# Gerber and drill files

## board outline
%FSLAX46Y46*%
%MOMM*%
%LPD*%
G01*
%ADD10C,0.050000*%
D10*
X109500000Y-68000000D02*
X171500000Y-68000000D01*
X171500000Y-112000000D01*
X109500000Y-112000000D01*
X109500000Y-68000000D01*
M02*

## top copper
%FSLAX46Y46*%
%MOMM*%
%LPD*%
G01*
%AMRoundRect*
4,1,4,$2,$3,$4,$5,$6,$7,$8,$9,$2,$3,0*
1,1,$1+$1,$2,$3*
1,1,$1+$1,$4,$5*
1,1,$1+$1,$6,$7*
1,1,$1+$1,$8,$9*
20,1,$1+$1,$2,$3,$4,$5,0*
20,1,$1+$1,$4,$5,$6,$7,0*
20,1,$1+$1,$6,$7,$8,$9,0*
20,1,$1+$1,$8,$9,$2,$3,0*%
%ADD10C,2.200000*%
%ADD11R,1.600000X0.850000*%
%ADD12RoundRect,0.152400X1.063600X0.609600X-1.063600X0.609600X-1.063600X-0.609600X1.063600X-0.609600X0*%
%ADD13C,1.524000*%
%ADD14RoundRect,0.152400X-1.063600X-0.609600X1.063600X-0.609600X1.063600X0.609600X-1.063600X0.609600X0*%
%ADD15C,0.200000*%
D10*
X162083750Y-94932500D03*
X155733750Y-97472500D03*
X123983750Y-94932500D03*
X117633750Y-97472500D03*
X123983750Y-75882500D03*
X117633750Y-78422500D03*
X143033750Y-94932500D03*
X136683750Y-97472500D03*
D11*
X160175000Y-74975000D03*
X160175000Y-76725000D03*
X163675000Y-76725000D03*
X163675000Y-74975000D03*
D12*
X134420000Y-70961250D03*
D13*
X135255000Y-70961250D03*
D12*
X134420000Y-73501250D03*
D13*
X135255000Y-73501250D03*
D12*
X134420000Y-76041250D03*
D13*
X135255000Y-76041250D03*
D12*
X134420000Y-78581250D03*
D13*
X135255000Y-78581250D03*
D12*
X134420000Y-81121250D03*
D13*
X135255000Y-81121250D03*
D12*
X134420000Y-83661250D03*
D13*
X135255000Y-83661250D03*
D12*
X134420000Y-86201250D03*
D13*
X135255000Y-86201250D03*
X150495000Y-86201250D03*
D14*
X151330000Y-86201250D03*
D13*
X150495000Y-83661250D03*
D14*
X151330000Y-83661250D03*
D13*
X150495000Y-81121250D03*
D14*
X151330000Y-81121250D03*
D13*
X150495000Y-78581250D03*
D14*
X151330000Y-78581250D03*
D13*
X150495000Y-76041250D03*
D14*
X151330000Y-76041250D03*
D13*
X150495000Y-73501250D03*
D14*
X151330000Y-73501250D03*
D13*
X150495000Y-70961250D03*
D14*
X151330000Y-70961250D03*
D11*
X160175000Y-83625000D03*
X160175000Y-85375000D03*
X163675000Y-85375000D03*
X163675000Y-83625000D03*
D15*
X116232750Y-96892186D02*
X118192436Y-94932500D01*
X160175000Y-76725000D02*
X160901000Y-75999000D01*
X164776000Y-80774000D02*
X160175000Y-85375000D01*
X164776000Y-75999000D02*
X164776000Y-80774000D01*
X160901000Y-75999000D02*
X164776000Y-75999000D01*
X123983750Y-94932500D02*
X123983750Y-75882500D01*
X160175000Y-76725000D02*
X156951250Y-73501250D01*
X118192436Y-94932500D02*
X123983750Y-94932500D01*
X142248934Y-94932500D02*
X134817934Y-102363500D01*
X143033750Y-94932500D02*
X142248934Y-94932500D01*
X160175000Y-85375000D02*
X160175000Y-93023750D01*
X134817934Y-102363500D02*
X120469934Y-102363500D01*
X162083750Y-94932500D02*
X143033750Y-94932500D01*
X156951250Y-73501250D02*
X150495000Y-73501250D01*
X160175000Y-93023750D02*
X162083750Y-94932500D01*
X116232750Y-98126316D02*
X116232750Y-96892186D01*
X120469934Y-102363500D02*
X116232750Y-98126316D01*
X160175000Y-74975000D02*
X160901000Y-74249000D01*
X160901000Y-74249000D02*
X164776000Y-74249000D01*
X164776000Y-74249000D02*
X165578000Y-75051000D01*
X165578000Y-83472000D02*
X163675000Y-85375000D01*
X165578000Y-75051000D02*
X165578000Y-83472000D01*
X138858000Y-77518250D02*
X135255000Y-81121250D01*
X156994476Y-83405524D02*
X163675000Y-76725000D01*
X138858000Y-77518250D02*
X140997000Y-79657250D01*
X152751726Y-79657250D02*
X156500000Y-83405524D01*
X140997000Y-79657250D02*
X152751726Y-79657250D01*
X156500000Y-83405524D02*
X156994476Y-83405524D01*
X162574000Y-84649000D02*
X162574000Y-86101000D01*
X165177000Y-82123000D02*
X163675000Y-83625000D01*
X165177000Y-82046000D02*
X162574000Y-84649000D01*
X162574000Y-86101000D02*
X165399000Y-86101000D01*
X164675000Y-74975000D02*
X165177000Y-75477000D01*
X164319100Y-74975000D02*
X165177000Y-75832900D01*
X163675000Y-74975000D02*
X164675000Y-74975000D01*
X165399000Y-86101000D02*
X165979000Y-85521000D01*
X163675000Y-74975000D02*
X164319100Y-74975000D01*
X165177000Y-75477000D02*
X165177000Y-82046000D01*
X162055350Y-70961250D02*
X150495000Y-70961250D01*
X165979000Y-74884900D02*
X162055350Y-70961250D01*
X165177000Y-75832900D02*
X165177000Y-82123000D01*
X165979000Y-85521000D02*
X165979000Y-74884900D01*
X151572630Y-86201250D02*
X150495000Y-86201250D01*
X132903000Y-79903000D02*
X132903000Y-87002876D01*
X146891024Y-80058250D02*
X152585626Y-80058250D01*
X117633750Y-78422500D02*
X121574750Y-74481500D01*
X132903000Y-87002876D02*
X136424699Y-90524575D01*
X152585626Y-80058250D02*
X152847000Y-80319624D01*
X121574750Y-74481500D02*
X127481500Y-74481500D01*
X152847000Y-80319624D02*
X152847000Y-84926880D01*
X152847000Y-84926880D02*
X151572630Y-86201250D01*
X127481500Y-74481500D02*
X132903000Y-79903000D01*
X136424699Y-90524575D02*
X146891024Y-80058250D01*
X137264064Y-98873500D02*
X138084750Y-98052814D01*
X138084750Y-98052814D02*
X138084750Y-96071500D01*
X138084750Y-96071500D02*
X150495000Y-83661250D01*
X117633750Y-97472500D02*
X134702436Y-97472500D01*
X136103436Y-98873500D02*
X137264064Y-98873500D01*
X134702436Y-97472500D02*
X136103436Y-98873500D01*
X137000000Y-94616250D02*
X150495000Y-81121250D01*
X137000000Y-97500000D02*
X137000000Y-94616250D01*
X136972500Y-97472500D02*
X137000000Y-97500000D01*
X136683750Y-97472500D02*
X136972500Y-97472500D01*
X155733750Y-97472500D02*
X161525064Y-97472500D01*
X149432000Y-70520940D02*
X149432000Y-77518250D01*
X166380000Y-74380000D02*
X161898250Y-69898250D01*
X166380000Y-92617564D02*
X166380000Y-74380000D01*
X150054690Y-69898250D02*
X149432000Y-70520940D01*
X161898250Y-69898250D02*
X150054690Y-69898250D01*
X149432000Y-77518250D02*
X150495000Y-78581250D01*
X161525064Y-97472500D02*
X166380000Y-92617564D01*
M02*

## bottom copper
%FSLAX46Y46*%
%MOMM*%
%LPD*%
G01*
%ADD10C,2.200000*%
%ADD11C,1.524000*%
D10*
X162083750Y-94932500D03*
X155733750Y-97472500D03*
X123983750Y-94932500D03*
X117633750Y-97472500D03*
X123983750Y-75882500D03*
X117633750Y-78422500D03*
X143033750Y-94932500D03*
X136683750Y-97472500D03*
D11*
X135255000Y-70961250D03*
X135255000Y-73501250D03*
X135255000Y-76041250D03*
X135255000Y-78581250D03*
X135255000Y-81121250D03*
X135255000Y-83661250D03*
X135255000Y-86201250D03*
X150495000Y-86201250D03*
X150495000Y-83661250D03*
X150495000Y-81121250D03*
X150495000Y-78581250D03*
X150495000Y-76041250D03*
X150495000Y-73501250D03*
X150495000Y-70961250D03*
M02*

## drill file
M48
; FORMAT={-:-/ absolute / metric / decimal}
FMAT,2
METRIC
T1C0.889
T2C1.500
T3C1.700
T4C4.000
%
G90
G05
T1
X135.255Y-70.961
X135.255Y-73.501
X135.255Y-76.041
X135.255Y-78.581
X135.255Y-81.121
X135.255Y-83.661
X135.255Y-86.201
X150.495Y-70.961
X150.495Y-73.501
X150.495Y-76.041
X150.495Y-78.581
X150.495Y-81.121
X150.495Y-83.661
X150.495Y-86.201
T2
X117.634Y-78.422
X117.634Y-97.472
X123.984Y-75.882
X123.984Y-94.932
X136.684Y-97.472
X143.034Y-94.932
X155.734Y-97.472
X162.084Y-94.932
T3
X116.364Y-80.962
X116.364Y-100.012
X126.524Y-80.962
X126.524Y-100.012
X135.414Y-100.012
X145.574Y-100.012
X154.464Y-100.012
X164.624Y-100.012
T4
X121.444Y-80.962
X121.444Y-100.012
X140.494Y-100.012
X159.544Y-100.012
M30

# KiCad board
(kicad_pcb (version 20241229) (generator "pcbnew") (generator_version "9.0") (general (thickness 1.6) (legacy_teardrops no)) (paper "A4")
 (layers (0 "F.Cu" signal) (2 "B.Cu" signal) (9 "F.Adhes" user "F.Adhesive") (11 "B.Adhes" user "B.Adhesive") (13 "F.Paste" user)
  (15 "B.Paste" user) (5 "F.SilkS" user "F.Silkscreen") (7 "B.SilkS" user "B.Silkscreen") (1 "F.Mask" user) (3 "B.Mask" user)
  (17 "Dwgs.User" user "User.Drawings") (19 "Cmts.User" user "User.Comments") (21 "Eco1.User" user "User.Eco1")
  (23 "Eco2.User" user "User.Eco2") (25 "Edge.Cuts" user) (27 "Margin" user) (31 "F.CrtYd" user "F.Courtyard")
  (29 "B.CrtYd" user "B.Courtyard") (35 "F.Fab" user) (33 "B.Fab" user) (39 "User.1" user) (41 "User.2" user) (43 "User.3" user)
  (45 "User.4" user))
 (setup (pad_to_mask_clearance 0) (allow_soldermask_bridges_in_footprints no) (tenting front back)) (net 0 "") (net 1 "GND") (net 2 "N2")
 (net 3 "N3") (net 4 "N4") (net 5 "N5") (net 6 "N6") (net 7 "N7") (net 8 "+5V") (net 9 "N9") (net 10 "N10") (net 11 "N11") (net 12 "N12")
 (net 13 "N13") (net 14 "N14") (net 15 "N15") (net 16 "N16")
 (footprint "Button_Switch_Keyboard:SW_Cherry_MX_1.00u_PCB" (layer "F.Cu") (at 162.08375 94.9325)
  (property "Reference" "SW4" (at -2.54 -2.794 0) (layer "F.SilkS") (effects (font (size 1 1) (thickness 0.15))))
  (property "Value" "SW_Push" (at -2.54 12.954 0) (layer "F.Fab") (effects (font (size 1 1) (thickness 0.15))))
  (pad "" np_thru_hole circle (at -7.62 5.08) (size 1.7 1.7) (drill 1.7) (layers "*.Cu" "*.Mask"))
  (pad "" np_thru_hole circle (at -2.54 5.08) (size 4 4) (drill 4) (layers "*.Cu" "*.Mask"))
  (pad "" np_thru_hole circle (at 2.54 5.08) (size 1.7 1.7) (drill 1.7) (layers "*.Cu" "*.Mask"))
  (pad "1" thru_hole circle (at 0 0) (size 2.2 2.2) (drill 1.5) (layers "*.Cu" "*.Mask") (remove_unused_layers no) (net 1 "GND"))
  (pad "2" thru_hole circle (at -6.35 2.54) (size 2.2 2.2) (drill 1.5) (layers "*.Cu" "*.Mask") (remove_unused_layers no) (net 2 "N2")))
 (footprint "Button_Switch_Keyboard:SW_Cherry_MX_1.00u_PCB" (layer "F.Cu") (at 123.98375 94.9325)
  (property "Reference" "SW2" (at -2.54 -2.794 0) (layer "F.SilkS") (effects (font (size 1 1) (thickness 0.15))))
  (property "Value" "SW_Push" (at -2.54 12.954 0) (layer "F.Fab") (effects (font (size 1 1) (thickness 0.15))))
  (pad "" np_thru_hole circle (at -7.62 5.08) (size 1.7 1.7) (drill 1.7) (layers "*.Cu" "*.Mask"))
  (pad "" np_thru_hole circle (at -2.54 5.08) (size 4 4) (drill 4) (layers "*.Cu" "*.Mask"))
  (pad "" np_thru_hole circle (at 2.54 5.08) (size 1.7 1.7) (drill 1.7) (layers "*.Cu" "*.Mask"))
  (pad "1" thru_hole circle (at 0 0) (size 2.2 2.2) (drill 1.5) (layers "*.Cu" "*.Mask") (remove_unused_layers no) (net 1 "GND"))
  (pad "2" thru_hole circle (at -6.35 2.54) (size 2.2 2.2) (drill 1.5) (layers "*.Cu" "*.Mask") (remove_unused_layers no) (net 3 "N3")))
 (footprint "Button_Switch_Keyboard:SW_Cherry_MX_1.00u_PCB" (layer "F.Cu") (at 123.98375 75.8825)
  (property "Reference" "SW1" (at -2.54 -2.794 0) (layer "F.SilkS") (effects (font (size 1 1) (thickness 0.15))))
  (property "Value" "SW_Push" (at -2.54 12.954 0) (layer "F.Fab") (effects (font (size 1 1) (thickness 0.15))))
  (pad "" np_thru_hole circle (at -7.62 5.08) (size 1.7 1.7) (drill 1.7) (layers "*.Cu" "*.Mask"))
  (pad "" np_thru_hole circle (at -2.54 5.08) (size 4 4) (drill 4) (layers "*.Cu" "*.Mask"))
  (pad "" np_thru_hole circle (at 2.54 5.08) (size 1.7 1.7) (drill 1.7) (layers "*.Cu" "*.Mask"))
  (pad "1" thru_hole circle (at 0 0) (size 2.2 2.2) (drill 1.5) (layers "*.Cu" "*.Mask") (remove_unused_layers no) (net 1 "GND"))
  (pad "2" thru_hole circle (at -6.35 2.54) (size 2.2 2.2) (drill 1.5) (layers "*.Cu" "*.Mask") (remove_unused_layers no) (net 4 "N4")))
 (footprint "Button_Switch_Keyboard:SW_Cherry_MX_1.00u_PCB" (layer "F.Cu") (at 143.03375 94.9325)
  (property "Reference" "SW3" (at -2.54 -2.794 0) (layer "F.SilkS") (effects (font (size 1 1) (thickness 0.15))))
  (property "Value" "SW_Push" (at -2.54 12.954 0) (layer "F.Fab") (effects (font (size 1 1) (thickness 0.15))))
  (pad "" np_thru_hole circle (at -7.62 5.08) (size 1.7 1.7) (drill 1.7) (layers "*.Cu" "*.Mask"))
  (pad "" np_thru_hole circle (at -2.54 5.08) (size 4 4) (drill 4) (layers "*.Cu" "*.Mask"))
  (pad "" np_thru_hole circle (at 2.54 5.08) (size 1.7 1.7) (drill 1.7) (layers "*.Cu" "*.Mask"))
  (pad "1" thru_hole circle (at 0 0) (size 2.2 2.2) (drill 1.5) (layers "*.Cu" "*.Mask") (remove_unused_layers no) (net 1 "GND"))
  (pad "2" thru_hole circle (at -6.35 2.54) (size 2.2 2.2) (drill 1.5) (layers "*.Cu" "*.Mask") (remove_unused_layers no) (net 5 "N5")))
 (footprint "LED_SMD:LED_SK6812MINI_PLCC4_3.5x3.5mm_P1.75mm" (layer "F.Cu") (at 161.925 75.85)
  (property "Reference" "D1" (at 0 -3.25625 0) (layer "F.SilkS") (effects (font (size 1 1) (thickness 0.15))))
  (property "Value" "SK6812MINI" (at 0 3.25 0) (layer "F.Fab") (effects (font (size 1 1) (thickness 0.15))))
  (pad "1" smd rect (at -1.75 -0.875) (size 1.6 0.85) (layers "F.Cu" "F.Mask" "F.Paste") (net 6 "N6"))
  (pad "2" smd rect (at -1.75 0.875) (size 1.6 0.85) (layers "F.Cu" "F.Mask" "F.Paste") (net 1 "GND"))
  (pad "3" smd rect (at 1.75 0.875) (size 1.6 0.85) (layers "F.Cu" "F.Mask" "F.Paste") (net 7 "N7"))
  (pad "4" smd rect (at 1.75 -0.875) (size 1.6 0.85) (layers "F.Cu" "F.Mask" "F.Paste") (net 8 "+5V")))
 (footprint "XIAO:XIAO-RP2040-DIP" (layer "F.Cu") (at 142.875 78.58125)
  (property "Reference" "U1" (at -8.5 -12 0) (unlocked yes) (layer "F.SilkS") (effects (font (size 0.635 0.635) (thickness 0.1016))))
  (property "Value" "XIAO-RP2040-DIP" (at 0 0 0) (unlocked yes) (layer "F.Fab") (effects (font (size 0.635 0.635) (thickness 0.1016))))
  (pad "1" smd roundrect (at -8.455 -7.62 180) (size 2.432 1.524) (layers "F.Cu" "F.Mask") (roundrect_rratio 0.1) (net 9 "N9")
   (thermal_bridge_angle 45))
  (pad "1" thru_hole circle (at -7.62 -7.62 180) (size 1.524 1.524) (drill 0.889) (layers "*.Cu" "*.Mask") (remove_unused_layers no)
   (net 9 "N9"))
  (pad "2" smd roundrect (at -8.455 -5.08 180) (size 2.432 1.524) (layers "F.Cu" "F.Mask") (roundrect_rratio 0.1) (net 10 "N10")
   (thermal_bridge_angle 45))
  (pad "2" thru_hole circle (at -7.62 -5.08 180) (size 1.524 1.524) (drill 0.889) (layers "*.Cu" "*.Mask") (remove_unused_layers no)
   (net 10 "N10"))
  (pad "3" smd roundrect (at -8.455 -2.54 180) (size 2.432 1.524) (layers "F.Cu" "F.Mask") (roundrect_rratio 0.1) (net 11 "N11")
   (thermal_bridge_angle 45))
  (pad "3" thru_hole circle (at -7.62 -2.54 180) (size 1.524 1.524) (drill 0.889) (layers "*.Cu" "*.Mask") (remove_unused_layers no)
   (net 11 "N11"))
  (pad "4" smd roundrect (at -8.455 0 180) (size 2.432 1.524) (layers "F.Cu" "F.Mask") (roundrect_rratio 0.1) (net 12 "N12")
   (thermal_bridge_angle 45))
  (pad "4" thru_hole circle (at -7.62 0 180) (size 1.524 1.524) (drill 0.889) (layers "*.Cu" "*.Mask") (remove_unused_layers no)
   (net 12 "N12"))
  (pad "5" smd roundrect (at -8.455 2.54 180) (size 2.432 1.524) (layers "F.Cu" "F.Mask") (roundrect_rratio 0.1) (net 7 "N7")
   (thermal_bridge_angle 45))
  (pad "5" thru_hole circle (at -7.62 2.54 180) (size 1.524 1.524) (drill 0.889) (layers "*.Cu" "*.Mask") (remove_unused_layers no)
   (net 7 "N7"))
  (pad "6" smd roundrect (at -8.455 5.08 180) (size 2.432 1.524) (layers "F.Cu" "F.Mask") (roundrect_rratio 0.1) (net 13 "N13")
   (thermal_bridge_angle 45))
  (pad "6" thru_hole circle (at -7.62 5.08 180) (size 1.524 1.524) (drill 0.889) (layers "*.Cu" "*.Mask") (remove_unused_layers no)
   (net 13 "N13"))
  (pad "7" smd roundrect (at -8.455 7.62 180) (size 2.432 1.524) (layers "F.Cu" "F.Mask") (roundrect_rratio 0.1) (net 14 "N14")
   (thermal_bridge_angle 45))
  (pad "7" thru_hole circle (at -7.62 7.62 180) (size 1.524 1.524) (drill 0.889) (layers "*.Cu" "*.Mask") (remove_unused_layers no)
   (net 14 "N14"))
  (pad "8" thru_hole circle (at 7.62 7.62) (size 1.524 1.524) (drill 0.889) (layers "*.Cu" "*.Mask") (remove_unused_layers no) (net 4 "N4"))
  (pad "8" smd roundrect (at 8.455 7.62) (size 2.432 1.524) (layers "F.Cu" "F.Mask") (roundrect_rratio 0.1) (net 4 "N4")
   (thermal_bridge_angle 45))
  (pad "9" thru_hole circle (at 7.62 5.08) (size 1.524 1.524) (drill 0.889) (layers "*.Cu" "*.Mask") (remove_unused_layers no) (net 3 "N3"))
  (pad "9" smd roundrect (at 8.455 5.08) (size 2.432 1.524) (layers "F.Cu" "F.Mask") (roundrect_rratio 0.1) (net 3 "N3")
   (thermal_bridge_angle 45))
  (pad "10" thru_hole circle (at 7.62 2.54) (size 1.524 1.524) (drill 0.889) (layers "*.Cu" "*.Mask") (remove_unused_layers no) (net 5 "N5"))
  (pad "10" smd roundrect (at 8.455 2.54) (size 2.432 1.524) (layers "F.Cu" "F.Mask") (roundrect_rratio 0.1) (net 5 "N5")
   (thermal_bridge_angle 45))
  (pad "11" thru_hole circle (at 7.62 0) (size 1.524 1.524) (drill 0.889) (layers "*.Cu" "*.Mask") (remove_unused_layers no) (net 2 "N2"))
  (pad "11" smd roundrect (at 8.455 0) (size 2.432 1.524) (layers "F.Cu" "F.Mask") (roundrect_rratio 0.1) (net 2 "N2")
   (thermal_bridge_angle 45))
  (pad "12" thru_hole circle (at 7.62 -2.54) (size 1.524 1.524) (drill 0.889) (layers "*.Cu" "*.Mask") (remove_unused_layers no)
   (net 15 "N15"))
  (pad "12" smd roundrect (at 8.455 -2.54) (size 2.432 1.524) (layers "F.Cu" "F.Mask") (roundrect_rratio 0.1) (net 15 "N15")
   (thermal_bridge_angle 45))
  (pad "13" thru_hole circle (at 7.62 -5.08) (size 1.524 1.524) (drill 0.889) (layers "*.Cu" "*.Mask") (remove_unused_layers no)
   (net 1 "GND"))
  (pad "13" smd roundrect (at 8.455 -5.08) (size 2.432 1.524) (layers "F.Cu" "F.Mask") (roundrect_rratio 0.1) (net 1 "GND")
   (thermal_bridge_angle 45))
  (pad "14" thru_hole circle (at 7.62 -7.62) (size 1.524 1.524) (drill 0.889) (layers "*.Cu" "*.Mask") (remove_unused_layers no)
   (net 8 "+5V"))
  (pad "14" smd roundrect (at 8.455 -7.62) (size 2.432 1.524) (layers "F.Cu" "F.Mask") (roundrect_rratio 0.1) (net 8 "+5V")
   (thermal_bridge_angle 45)))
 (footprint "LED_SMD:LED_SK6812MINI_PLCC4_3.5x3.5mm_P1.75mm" (layer "F.Cu") (at 161.925 84.5)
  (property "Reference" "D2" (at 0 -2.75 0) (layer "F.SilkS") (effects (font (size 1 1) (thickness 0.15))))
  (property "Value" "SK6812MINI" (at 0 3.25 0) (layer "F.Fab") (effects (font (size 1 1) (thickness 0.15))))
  (pad "1" smd rect (at -1.75 -0.875) (size 1.6 0.85) (layers "F.Cu" "F.Mask" "F.Paste") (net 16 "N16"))
  (pad "2" smd rect (at -1.75 0.875) (size 1.6 0.85) (layers "F.Cu" "F.Mask" "F.Paste") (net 1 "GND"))
  (pad "3" smd rect (at 1.75 0.875) (size 1.6 0.85) (layers "F.Cu" "F.Mask" "F.Paste") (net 6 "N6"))
  (pad "4" smd rect (at 1.75 -0.875) (size 1.6 0.85) (layers "F.Cu" "F.Mask" "F.Paste") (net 8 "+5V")))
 (gr_rect (start 109.5 68) (end 171.5 112) (stroke (width 0.05) (type default)) (fill no) (layer "Edge.Cuts"))
 (segment (start 116.23275 96.892186) (end 118.192436 94.9325) (width 0.2) (layer "F.Cu") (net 1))
 (segment (start 160.175 76.725) (end 160.901 75.999) (width 0.2) (layer "F.Cu") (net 1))
 (segment (start 164.776 80.774) (end 160.175 85.375) (width 0.2) (layer "F.Cu") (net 1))
 (segment (start 164.776 75.999) (end 164.776 80.774) (width 0.2) (layer "F.Cu") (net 1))
 (segment (start 160.901 75.999) (end 164.776 75.999) (width 0.2) (layer "F.Cu") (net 1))
 (segment (start 123.98375 94.9325) (end 123.98375 75.8825) (width 0.2) (layer "F.Cu") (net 1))
 (segment (start 160.175 76.725) (end 156.95125 73.50125) (width 0.2) (layer "F.Cu") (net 1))
 (segment (start 118.192436 94.9325) (end 123.98375 94.9325) (width 0.2) (layer "F.Cu") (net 1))
 (segment (start 142.248934 94.9325) (end 134.817934 102.3635) (width 0.2) (layer "F.Cu") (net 1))
 (segment (start 143.03375 94.9325) (end 142.248934 94.9325) (width 0.2) (layer "F.Cu") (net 1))
 (segment (start 160.175 85.375) (end 160.175 93.02375) (width 0.2) (layer "F.Cu") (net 1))
 (segment (start 134.817934 102.3635) (end 120.469934 102.3635) (width 0.2) (layer "F.Cu") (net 1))
 (segment (start 162.08375 94.9325) (end 143.03375 94.9325) (width 0.2) (layer "F.Cu") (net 1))
 (segment (start 156.95125 73.50125) (end 150.495 73.50125) (width 0.2) (layer "F.Cu") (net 1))
 (segment (start 160.175 93.02375) (end 162.08375 94.9325) (width 0.2) (layer "F.Cu") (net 1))
 (segment (start 116.23275 98.126316) (end 116.23275 96.892186) (width 0.2) (layer "F.Cu") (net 1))
 (segment (start 120.469934 102.3635) (end 116.23275 98.126316) (width 0.2) (layer "F.Cu") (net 1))
 (segment (start 160.175 74.975) (end 160.901 74.249) (width 0.2) (layer "F.Cu") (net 6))
 (segment (start 160.901 74.249) (end 164.776 74.249) (width 0.2) (layer "F.Cu") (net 6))
 (segment (start 164.776 74.249) (end 165.578 75.051) (width 0.2) (layer "F.Cu") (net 6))
 (segment (start 165.578 83.472) (end 163.675 85.375) (width 0.2) (layer "F.Cu") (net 6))
 (segment (start 165.578 75.051) (end 165.578 83.472) (width 0.2) (layer "F.Cu") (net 6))
 (segment (start 138.858 77.51825) (end 135.255 81.12125) (width 0.2) (layer "F.Cu") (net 7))
 (segment (start 156.994476 83.405524) (end 163.675 76.725) (width 0.2) (layer "F.Cu") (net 7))
 (segment (start 138.858 77.51825) (end 140.997 79.65725) (width 0.2) (layer "F.Cu") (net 7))
 (segment (start 152.751726 79.65725) (end 156.5 83.405524) (width 0.2) (layer "F.Cu") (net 7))
 (segment (start 140.997 79.65725) (end 152.751726 79.65725) (width 0.2) (layer "F.Cu") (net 7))
 (segment (start 156.5 83.405524) (end 156.994476 83.405524) (width 0.2) (layer "F.Cu") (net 7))
 (segment (start 162.574 84.649) (end 162.574 86.101) (width 0.2) (layer "F.Cu") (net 8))
 (segment (start 165.177 82.123) (end 163.675 83.625) (width 0.2) (layer "F.Cu") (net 8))
 (segment (start 165.177 82.046) (end 162.574 84.649) (width 0.2) (layer "F.Cu") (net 8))
 (segment (start 162.574 86.101) (end 165.399 86.101) (width 0.2) (layer "F.Cu") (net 8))
 (segment (start 164.675 74.975) (end 165.177 75.477) (width 0.2) (layer "F.Cu") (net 8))
 (segment (start 164.3191 74.975) (end 165.177 75.8329) (width 0.2) (layer "F.Cu") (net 8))
 (segment (start 163.675 74.975) (end 164.675 74.975) (width 0.2) (layer "F.Cu") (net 8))
 (segment (start 165.399 86.101) (end 165.979 85.521) (width 0.2) (layer "F.Cu") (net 8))
 (segment (start 163.675 74.975) (end 164.3191 74.975) (width 0.2) (layer "F.Cu") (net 8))
 (segment (start 165.177 75.477) (end 165.177 82.046) (width 0.2) (layer "F.Cu") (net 8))
 (segment (start 162.05535 70.96125) (end 150.495 70.96125) (width 0.2) (layer "F.Cu") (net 8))
 (segment (start 165.979 74.8849) (end 162.05535 70.96125) (width 0.2) (layer "F.Cu") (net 8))
 (segment (start 165.177 75.8329) (end 165.177 82.123) (width 0.2) (layer "F.Cu") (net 8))
 (segment (start 165.979 85.521) (end 165.979 74.8849) (width 0.2) (layer "F.Cu") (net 8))
 (segment (start 151.57263 86.20125) (end 150.495 86.20125) (width 0.2) (layer "F.Cu") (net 4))
 (segment (start 132.903 79.903) (end 132.903 87.002876) (width 0.2) (layer "F.Cu") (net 4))
 (segment (start 146.891024 80.05825) (end 152.585626 80.05825) (width 0.2) (layer "F.Cu") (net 4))
 (segment (start 117.63375 78.4225) (end 121.57475 74.4815) (width 0.2) (layer "F.Cu") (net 4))
 (segment (start 132.903 87.002876) (end 136.424699 90.524575) (width 0.2) (layer "F.Cu") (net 4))
 (segment (start 152.585626 80.05825) (end 152.847 80.319624) (width 0.2) (layer "F.Cu") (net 4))
 (segment (start 121.57475 74.4815) (end 127.4815 74.4815) (width 0.2) (layer "F.Cu") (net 4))
 (segment (start 152.847 80.319624) (end 152.847 84.92688) (width 0.2) (layer "F.Cu") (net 4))
 (segment (start 152.847 84.92688) (end 151.57263 86.20125) (width 0.2) (layer "F.Cu") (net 4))
 (segment (start 127.4815 74.4815) (end 132.903 79.903) (width 0.2) (layer "F.Cu") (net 4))
 (segment (start 136.424699 90.524575) (end 146.891024 80.05825) (width 0.2) (layer "F.Cu") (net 4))
 (segment (start 137.264064 98.8735) (end 138.08475 98.052814) (width 0.2) (layer "F.Cu") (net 3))
 (segment (start 138.08475 98.052814) (end 138.08475 96.0715) (width 0.2) (layer "F.Cu") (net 3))
 (segment (start 138.08475 96.0715) (end 150.495 83.66125) (width 0.2) (layer "F.Cu") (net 3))
 (segment (start 117.63375 97.4725) (end 134.702436 97.4725) (width 0.2) (layer "F.Cu") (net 3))
 (segment (start 136.103436 98.8735) (end 137.264064 98.8735) (width 0.2) (layer "F.Cu") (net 3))
 (segment (start 134.702436 97.4725) (end 136.103436 98.8735) (width 0.2) (layer "F.Cu") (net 3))
 (segment (start 137 94.61625) (end 150.495 81.12125) (width 0.2) (layer "F.Cu") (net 5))
 (segment (start 137 97.5) (end 137 94.61625) (width 0.2) (layer "F.Cu") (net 5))
 (segment (start 136.9725 97.4725) (end 137 97.5) (width 0.2) (layer "F.Cu") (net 5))
 (segment (start 136.68375 97.4725) (end 136.9725 97.4725) (width 0.2) (layer "F.Cu") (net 5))
 (segment (start 155.73375 97.4725) (end 161.525064 97.4725) (width 0.2) (layer "F.Cu") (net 2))
 (segment (start 149.432 70.52094) (end 149.432 77.51825) (width 0.2) (layer "F.Cu") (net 2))
 (segment (start 166.38 74.38) (end 161.89825 69.89825) (width 0.2) (layer "F.Cu") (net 2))
 (segment (start 166.38 92.617564) (end 166.38 74.38) (width 0.2) (layer "F.Cu") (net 2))
 (segment (start 150.05469 69.89825) (end 149.432 70.52094) (width 0.2) (layer "F.Cu") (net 2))
 (segment (start 161.89825 69.89825) (end 150.05469 69.89825) (width 0.2) (layer "F.Cu") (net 2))
 (segment (start 149.432 77.51825) (end 150.495 78.58125) (width 0.2) (layer "F.Cu") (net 2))
 (segment (start 161.525064 97.4725) (end 166.38 92.617564) (width 0.2) (layer "F.Cu") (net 2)))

